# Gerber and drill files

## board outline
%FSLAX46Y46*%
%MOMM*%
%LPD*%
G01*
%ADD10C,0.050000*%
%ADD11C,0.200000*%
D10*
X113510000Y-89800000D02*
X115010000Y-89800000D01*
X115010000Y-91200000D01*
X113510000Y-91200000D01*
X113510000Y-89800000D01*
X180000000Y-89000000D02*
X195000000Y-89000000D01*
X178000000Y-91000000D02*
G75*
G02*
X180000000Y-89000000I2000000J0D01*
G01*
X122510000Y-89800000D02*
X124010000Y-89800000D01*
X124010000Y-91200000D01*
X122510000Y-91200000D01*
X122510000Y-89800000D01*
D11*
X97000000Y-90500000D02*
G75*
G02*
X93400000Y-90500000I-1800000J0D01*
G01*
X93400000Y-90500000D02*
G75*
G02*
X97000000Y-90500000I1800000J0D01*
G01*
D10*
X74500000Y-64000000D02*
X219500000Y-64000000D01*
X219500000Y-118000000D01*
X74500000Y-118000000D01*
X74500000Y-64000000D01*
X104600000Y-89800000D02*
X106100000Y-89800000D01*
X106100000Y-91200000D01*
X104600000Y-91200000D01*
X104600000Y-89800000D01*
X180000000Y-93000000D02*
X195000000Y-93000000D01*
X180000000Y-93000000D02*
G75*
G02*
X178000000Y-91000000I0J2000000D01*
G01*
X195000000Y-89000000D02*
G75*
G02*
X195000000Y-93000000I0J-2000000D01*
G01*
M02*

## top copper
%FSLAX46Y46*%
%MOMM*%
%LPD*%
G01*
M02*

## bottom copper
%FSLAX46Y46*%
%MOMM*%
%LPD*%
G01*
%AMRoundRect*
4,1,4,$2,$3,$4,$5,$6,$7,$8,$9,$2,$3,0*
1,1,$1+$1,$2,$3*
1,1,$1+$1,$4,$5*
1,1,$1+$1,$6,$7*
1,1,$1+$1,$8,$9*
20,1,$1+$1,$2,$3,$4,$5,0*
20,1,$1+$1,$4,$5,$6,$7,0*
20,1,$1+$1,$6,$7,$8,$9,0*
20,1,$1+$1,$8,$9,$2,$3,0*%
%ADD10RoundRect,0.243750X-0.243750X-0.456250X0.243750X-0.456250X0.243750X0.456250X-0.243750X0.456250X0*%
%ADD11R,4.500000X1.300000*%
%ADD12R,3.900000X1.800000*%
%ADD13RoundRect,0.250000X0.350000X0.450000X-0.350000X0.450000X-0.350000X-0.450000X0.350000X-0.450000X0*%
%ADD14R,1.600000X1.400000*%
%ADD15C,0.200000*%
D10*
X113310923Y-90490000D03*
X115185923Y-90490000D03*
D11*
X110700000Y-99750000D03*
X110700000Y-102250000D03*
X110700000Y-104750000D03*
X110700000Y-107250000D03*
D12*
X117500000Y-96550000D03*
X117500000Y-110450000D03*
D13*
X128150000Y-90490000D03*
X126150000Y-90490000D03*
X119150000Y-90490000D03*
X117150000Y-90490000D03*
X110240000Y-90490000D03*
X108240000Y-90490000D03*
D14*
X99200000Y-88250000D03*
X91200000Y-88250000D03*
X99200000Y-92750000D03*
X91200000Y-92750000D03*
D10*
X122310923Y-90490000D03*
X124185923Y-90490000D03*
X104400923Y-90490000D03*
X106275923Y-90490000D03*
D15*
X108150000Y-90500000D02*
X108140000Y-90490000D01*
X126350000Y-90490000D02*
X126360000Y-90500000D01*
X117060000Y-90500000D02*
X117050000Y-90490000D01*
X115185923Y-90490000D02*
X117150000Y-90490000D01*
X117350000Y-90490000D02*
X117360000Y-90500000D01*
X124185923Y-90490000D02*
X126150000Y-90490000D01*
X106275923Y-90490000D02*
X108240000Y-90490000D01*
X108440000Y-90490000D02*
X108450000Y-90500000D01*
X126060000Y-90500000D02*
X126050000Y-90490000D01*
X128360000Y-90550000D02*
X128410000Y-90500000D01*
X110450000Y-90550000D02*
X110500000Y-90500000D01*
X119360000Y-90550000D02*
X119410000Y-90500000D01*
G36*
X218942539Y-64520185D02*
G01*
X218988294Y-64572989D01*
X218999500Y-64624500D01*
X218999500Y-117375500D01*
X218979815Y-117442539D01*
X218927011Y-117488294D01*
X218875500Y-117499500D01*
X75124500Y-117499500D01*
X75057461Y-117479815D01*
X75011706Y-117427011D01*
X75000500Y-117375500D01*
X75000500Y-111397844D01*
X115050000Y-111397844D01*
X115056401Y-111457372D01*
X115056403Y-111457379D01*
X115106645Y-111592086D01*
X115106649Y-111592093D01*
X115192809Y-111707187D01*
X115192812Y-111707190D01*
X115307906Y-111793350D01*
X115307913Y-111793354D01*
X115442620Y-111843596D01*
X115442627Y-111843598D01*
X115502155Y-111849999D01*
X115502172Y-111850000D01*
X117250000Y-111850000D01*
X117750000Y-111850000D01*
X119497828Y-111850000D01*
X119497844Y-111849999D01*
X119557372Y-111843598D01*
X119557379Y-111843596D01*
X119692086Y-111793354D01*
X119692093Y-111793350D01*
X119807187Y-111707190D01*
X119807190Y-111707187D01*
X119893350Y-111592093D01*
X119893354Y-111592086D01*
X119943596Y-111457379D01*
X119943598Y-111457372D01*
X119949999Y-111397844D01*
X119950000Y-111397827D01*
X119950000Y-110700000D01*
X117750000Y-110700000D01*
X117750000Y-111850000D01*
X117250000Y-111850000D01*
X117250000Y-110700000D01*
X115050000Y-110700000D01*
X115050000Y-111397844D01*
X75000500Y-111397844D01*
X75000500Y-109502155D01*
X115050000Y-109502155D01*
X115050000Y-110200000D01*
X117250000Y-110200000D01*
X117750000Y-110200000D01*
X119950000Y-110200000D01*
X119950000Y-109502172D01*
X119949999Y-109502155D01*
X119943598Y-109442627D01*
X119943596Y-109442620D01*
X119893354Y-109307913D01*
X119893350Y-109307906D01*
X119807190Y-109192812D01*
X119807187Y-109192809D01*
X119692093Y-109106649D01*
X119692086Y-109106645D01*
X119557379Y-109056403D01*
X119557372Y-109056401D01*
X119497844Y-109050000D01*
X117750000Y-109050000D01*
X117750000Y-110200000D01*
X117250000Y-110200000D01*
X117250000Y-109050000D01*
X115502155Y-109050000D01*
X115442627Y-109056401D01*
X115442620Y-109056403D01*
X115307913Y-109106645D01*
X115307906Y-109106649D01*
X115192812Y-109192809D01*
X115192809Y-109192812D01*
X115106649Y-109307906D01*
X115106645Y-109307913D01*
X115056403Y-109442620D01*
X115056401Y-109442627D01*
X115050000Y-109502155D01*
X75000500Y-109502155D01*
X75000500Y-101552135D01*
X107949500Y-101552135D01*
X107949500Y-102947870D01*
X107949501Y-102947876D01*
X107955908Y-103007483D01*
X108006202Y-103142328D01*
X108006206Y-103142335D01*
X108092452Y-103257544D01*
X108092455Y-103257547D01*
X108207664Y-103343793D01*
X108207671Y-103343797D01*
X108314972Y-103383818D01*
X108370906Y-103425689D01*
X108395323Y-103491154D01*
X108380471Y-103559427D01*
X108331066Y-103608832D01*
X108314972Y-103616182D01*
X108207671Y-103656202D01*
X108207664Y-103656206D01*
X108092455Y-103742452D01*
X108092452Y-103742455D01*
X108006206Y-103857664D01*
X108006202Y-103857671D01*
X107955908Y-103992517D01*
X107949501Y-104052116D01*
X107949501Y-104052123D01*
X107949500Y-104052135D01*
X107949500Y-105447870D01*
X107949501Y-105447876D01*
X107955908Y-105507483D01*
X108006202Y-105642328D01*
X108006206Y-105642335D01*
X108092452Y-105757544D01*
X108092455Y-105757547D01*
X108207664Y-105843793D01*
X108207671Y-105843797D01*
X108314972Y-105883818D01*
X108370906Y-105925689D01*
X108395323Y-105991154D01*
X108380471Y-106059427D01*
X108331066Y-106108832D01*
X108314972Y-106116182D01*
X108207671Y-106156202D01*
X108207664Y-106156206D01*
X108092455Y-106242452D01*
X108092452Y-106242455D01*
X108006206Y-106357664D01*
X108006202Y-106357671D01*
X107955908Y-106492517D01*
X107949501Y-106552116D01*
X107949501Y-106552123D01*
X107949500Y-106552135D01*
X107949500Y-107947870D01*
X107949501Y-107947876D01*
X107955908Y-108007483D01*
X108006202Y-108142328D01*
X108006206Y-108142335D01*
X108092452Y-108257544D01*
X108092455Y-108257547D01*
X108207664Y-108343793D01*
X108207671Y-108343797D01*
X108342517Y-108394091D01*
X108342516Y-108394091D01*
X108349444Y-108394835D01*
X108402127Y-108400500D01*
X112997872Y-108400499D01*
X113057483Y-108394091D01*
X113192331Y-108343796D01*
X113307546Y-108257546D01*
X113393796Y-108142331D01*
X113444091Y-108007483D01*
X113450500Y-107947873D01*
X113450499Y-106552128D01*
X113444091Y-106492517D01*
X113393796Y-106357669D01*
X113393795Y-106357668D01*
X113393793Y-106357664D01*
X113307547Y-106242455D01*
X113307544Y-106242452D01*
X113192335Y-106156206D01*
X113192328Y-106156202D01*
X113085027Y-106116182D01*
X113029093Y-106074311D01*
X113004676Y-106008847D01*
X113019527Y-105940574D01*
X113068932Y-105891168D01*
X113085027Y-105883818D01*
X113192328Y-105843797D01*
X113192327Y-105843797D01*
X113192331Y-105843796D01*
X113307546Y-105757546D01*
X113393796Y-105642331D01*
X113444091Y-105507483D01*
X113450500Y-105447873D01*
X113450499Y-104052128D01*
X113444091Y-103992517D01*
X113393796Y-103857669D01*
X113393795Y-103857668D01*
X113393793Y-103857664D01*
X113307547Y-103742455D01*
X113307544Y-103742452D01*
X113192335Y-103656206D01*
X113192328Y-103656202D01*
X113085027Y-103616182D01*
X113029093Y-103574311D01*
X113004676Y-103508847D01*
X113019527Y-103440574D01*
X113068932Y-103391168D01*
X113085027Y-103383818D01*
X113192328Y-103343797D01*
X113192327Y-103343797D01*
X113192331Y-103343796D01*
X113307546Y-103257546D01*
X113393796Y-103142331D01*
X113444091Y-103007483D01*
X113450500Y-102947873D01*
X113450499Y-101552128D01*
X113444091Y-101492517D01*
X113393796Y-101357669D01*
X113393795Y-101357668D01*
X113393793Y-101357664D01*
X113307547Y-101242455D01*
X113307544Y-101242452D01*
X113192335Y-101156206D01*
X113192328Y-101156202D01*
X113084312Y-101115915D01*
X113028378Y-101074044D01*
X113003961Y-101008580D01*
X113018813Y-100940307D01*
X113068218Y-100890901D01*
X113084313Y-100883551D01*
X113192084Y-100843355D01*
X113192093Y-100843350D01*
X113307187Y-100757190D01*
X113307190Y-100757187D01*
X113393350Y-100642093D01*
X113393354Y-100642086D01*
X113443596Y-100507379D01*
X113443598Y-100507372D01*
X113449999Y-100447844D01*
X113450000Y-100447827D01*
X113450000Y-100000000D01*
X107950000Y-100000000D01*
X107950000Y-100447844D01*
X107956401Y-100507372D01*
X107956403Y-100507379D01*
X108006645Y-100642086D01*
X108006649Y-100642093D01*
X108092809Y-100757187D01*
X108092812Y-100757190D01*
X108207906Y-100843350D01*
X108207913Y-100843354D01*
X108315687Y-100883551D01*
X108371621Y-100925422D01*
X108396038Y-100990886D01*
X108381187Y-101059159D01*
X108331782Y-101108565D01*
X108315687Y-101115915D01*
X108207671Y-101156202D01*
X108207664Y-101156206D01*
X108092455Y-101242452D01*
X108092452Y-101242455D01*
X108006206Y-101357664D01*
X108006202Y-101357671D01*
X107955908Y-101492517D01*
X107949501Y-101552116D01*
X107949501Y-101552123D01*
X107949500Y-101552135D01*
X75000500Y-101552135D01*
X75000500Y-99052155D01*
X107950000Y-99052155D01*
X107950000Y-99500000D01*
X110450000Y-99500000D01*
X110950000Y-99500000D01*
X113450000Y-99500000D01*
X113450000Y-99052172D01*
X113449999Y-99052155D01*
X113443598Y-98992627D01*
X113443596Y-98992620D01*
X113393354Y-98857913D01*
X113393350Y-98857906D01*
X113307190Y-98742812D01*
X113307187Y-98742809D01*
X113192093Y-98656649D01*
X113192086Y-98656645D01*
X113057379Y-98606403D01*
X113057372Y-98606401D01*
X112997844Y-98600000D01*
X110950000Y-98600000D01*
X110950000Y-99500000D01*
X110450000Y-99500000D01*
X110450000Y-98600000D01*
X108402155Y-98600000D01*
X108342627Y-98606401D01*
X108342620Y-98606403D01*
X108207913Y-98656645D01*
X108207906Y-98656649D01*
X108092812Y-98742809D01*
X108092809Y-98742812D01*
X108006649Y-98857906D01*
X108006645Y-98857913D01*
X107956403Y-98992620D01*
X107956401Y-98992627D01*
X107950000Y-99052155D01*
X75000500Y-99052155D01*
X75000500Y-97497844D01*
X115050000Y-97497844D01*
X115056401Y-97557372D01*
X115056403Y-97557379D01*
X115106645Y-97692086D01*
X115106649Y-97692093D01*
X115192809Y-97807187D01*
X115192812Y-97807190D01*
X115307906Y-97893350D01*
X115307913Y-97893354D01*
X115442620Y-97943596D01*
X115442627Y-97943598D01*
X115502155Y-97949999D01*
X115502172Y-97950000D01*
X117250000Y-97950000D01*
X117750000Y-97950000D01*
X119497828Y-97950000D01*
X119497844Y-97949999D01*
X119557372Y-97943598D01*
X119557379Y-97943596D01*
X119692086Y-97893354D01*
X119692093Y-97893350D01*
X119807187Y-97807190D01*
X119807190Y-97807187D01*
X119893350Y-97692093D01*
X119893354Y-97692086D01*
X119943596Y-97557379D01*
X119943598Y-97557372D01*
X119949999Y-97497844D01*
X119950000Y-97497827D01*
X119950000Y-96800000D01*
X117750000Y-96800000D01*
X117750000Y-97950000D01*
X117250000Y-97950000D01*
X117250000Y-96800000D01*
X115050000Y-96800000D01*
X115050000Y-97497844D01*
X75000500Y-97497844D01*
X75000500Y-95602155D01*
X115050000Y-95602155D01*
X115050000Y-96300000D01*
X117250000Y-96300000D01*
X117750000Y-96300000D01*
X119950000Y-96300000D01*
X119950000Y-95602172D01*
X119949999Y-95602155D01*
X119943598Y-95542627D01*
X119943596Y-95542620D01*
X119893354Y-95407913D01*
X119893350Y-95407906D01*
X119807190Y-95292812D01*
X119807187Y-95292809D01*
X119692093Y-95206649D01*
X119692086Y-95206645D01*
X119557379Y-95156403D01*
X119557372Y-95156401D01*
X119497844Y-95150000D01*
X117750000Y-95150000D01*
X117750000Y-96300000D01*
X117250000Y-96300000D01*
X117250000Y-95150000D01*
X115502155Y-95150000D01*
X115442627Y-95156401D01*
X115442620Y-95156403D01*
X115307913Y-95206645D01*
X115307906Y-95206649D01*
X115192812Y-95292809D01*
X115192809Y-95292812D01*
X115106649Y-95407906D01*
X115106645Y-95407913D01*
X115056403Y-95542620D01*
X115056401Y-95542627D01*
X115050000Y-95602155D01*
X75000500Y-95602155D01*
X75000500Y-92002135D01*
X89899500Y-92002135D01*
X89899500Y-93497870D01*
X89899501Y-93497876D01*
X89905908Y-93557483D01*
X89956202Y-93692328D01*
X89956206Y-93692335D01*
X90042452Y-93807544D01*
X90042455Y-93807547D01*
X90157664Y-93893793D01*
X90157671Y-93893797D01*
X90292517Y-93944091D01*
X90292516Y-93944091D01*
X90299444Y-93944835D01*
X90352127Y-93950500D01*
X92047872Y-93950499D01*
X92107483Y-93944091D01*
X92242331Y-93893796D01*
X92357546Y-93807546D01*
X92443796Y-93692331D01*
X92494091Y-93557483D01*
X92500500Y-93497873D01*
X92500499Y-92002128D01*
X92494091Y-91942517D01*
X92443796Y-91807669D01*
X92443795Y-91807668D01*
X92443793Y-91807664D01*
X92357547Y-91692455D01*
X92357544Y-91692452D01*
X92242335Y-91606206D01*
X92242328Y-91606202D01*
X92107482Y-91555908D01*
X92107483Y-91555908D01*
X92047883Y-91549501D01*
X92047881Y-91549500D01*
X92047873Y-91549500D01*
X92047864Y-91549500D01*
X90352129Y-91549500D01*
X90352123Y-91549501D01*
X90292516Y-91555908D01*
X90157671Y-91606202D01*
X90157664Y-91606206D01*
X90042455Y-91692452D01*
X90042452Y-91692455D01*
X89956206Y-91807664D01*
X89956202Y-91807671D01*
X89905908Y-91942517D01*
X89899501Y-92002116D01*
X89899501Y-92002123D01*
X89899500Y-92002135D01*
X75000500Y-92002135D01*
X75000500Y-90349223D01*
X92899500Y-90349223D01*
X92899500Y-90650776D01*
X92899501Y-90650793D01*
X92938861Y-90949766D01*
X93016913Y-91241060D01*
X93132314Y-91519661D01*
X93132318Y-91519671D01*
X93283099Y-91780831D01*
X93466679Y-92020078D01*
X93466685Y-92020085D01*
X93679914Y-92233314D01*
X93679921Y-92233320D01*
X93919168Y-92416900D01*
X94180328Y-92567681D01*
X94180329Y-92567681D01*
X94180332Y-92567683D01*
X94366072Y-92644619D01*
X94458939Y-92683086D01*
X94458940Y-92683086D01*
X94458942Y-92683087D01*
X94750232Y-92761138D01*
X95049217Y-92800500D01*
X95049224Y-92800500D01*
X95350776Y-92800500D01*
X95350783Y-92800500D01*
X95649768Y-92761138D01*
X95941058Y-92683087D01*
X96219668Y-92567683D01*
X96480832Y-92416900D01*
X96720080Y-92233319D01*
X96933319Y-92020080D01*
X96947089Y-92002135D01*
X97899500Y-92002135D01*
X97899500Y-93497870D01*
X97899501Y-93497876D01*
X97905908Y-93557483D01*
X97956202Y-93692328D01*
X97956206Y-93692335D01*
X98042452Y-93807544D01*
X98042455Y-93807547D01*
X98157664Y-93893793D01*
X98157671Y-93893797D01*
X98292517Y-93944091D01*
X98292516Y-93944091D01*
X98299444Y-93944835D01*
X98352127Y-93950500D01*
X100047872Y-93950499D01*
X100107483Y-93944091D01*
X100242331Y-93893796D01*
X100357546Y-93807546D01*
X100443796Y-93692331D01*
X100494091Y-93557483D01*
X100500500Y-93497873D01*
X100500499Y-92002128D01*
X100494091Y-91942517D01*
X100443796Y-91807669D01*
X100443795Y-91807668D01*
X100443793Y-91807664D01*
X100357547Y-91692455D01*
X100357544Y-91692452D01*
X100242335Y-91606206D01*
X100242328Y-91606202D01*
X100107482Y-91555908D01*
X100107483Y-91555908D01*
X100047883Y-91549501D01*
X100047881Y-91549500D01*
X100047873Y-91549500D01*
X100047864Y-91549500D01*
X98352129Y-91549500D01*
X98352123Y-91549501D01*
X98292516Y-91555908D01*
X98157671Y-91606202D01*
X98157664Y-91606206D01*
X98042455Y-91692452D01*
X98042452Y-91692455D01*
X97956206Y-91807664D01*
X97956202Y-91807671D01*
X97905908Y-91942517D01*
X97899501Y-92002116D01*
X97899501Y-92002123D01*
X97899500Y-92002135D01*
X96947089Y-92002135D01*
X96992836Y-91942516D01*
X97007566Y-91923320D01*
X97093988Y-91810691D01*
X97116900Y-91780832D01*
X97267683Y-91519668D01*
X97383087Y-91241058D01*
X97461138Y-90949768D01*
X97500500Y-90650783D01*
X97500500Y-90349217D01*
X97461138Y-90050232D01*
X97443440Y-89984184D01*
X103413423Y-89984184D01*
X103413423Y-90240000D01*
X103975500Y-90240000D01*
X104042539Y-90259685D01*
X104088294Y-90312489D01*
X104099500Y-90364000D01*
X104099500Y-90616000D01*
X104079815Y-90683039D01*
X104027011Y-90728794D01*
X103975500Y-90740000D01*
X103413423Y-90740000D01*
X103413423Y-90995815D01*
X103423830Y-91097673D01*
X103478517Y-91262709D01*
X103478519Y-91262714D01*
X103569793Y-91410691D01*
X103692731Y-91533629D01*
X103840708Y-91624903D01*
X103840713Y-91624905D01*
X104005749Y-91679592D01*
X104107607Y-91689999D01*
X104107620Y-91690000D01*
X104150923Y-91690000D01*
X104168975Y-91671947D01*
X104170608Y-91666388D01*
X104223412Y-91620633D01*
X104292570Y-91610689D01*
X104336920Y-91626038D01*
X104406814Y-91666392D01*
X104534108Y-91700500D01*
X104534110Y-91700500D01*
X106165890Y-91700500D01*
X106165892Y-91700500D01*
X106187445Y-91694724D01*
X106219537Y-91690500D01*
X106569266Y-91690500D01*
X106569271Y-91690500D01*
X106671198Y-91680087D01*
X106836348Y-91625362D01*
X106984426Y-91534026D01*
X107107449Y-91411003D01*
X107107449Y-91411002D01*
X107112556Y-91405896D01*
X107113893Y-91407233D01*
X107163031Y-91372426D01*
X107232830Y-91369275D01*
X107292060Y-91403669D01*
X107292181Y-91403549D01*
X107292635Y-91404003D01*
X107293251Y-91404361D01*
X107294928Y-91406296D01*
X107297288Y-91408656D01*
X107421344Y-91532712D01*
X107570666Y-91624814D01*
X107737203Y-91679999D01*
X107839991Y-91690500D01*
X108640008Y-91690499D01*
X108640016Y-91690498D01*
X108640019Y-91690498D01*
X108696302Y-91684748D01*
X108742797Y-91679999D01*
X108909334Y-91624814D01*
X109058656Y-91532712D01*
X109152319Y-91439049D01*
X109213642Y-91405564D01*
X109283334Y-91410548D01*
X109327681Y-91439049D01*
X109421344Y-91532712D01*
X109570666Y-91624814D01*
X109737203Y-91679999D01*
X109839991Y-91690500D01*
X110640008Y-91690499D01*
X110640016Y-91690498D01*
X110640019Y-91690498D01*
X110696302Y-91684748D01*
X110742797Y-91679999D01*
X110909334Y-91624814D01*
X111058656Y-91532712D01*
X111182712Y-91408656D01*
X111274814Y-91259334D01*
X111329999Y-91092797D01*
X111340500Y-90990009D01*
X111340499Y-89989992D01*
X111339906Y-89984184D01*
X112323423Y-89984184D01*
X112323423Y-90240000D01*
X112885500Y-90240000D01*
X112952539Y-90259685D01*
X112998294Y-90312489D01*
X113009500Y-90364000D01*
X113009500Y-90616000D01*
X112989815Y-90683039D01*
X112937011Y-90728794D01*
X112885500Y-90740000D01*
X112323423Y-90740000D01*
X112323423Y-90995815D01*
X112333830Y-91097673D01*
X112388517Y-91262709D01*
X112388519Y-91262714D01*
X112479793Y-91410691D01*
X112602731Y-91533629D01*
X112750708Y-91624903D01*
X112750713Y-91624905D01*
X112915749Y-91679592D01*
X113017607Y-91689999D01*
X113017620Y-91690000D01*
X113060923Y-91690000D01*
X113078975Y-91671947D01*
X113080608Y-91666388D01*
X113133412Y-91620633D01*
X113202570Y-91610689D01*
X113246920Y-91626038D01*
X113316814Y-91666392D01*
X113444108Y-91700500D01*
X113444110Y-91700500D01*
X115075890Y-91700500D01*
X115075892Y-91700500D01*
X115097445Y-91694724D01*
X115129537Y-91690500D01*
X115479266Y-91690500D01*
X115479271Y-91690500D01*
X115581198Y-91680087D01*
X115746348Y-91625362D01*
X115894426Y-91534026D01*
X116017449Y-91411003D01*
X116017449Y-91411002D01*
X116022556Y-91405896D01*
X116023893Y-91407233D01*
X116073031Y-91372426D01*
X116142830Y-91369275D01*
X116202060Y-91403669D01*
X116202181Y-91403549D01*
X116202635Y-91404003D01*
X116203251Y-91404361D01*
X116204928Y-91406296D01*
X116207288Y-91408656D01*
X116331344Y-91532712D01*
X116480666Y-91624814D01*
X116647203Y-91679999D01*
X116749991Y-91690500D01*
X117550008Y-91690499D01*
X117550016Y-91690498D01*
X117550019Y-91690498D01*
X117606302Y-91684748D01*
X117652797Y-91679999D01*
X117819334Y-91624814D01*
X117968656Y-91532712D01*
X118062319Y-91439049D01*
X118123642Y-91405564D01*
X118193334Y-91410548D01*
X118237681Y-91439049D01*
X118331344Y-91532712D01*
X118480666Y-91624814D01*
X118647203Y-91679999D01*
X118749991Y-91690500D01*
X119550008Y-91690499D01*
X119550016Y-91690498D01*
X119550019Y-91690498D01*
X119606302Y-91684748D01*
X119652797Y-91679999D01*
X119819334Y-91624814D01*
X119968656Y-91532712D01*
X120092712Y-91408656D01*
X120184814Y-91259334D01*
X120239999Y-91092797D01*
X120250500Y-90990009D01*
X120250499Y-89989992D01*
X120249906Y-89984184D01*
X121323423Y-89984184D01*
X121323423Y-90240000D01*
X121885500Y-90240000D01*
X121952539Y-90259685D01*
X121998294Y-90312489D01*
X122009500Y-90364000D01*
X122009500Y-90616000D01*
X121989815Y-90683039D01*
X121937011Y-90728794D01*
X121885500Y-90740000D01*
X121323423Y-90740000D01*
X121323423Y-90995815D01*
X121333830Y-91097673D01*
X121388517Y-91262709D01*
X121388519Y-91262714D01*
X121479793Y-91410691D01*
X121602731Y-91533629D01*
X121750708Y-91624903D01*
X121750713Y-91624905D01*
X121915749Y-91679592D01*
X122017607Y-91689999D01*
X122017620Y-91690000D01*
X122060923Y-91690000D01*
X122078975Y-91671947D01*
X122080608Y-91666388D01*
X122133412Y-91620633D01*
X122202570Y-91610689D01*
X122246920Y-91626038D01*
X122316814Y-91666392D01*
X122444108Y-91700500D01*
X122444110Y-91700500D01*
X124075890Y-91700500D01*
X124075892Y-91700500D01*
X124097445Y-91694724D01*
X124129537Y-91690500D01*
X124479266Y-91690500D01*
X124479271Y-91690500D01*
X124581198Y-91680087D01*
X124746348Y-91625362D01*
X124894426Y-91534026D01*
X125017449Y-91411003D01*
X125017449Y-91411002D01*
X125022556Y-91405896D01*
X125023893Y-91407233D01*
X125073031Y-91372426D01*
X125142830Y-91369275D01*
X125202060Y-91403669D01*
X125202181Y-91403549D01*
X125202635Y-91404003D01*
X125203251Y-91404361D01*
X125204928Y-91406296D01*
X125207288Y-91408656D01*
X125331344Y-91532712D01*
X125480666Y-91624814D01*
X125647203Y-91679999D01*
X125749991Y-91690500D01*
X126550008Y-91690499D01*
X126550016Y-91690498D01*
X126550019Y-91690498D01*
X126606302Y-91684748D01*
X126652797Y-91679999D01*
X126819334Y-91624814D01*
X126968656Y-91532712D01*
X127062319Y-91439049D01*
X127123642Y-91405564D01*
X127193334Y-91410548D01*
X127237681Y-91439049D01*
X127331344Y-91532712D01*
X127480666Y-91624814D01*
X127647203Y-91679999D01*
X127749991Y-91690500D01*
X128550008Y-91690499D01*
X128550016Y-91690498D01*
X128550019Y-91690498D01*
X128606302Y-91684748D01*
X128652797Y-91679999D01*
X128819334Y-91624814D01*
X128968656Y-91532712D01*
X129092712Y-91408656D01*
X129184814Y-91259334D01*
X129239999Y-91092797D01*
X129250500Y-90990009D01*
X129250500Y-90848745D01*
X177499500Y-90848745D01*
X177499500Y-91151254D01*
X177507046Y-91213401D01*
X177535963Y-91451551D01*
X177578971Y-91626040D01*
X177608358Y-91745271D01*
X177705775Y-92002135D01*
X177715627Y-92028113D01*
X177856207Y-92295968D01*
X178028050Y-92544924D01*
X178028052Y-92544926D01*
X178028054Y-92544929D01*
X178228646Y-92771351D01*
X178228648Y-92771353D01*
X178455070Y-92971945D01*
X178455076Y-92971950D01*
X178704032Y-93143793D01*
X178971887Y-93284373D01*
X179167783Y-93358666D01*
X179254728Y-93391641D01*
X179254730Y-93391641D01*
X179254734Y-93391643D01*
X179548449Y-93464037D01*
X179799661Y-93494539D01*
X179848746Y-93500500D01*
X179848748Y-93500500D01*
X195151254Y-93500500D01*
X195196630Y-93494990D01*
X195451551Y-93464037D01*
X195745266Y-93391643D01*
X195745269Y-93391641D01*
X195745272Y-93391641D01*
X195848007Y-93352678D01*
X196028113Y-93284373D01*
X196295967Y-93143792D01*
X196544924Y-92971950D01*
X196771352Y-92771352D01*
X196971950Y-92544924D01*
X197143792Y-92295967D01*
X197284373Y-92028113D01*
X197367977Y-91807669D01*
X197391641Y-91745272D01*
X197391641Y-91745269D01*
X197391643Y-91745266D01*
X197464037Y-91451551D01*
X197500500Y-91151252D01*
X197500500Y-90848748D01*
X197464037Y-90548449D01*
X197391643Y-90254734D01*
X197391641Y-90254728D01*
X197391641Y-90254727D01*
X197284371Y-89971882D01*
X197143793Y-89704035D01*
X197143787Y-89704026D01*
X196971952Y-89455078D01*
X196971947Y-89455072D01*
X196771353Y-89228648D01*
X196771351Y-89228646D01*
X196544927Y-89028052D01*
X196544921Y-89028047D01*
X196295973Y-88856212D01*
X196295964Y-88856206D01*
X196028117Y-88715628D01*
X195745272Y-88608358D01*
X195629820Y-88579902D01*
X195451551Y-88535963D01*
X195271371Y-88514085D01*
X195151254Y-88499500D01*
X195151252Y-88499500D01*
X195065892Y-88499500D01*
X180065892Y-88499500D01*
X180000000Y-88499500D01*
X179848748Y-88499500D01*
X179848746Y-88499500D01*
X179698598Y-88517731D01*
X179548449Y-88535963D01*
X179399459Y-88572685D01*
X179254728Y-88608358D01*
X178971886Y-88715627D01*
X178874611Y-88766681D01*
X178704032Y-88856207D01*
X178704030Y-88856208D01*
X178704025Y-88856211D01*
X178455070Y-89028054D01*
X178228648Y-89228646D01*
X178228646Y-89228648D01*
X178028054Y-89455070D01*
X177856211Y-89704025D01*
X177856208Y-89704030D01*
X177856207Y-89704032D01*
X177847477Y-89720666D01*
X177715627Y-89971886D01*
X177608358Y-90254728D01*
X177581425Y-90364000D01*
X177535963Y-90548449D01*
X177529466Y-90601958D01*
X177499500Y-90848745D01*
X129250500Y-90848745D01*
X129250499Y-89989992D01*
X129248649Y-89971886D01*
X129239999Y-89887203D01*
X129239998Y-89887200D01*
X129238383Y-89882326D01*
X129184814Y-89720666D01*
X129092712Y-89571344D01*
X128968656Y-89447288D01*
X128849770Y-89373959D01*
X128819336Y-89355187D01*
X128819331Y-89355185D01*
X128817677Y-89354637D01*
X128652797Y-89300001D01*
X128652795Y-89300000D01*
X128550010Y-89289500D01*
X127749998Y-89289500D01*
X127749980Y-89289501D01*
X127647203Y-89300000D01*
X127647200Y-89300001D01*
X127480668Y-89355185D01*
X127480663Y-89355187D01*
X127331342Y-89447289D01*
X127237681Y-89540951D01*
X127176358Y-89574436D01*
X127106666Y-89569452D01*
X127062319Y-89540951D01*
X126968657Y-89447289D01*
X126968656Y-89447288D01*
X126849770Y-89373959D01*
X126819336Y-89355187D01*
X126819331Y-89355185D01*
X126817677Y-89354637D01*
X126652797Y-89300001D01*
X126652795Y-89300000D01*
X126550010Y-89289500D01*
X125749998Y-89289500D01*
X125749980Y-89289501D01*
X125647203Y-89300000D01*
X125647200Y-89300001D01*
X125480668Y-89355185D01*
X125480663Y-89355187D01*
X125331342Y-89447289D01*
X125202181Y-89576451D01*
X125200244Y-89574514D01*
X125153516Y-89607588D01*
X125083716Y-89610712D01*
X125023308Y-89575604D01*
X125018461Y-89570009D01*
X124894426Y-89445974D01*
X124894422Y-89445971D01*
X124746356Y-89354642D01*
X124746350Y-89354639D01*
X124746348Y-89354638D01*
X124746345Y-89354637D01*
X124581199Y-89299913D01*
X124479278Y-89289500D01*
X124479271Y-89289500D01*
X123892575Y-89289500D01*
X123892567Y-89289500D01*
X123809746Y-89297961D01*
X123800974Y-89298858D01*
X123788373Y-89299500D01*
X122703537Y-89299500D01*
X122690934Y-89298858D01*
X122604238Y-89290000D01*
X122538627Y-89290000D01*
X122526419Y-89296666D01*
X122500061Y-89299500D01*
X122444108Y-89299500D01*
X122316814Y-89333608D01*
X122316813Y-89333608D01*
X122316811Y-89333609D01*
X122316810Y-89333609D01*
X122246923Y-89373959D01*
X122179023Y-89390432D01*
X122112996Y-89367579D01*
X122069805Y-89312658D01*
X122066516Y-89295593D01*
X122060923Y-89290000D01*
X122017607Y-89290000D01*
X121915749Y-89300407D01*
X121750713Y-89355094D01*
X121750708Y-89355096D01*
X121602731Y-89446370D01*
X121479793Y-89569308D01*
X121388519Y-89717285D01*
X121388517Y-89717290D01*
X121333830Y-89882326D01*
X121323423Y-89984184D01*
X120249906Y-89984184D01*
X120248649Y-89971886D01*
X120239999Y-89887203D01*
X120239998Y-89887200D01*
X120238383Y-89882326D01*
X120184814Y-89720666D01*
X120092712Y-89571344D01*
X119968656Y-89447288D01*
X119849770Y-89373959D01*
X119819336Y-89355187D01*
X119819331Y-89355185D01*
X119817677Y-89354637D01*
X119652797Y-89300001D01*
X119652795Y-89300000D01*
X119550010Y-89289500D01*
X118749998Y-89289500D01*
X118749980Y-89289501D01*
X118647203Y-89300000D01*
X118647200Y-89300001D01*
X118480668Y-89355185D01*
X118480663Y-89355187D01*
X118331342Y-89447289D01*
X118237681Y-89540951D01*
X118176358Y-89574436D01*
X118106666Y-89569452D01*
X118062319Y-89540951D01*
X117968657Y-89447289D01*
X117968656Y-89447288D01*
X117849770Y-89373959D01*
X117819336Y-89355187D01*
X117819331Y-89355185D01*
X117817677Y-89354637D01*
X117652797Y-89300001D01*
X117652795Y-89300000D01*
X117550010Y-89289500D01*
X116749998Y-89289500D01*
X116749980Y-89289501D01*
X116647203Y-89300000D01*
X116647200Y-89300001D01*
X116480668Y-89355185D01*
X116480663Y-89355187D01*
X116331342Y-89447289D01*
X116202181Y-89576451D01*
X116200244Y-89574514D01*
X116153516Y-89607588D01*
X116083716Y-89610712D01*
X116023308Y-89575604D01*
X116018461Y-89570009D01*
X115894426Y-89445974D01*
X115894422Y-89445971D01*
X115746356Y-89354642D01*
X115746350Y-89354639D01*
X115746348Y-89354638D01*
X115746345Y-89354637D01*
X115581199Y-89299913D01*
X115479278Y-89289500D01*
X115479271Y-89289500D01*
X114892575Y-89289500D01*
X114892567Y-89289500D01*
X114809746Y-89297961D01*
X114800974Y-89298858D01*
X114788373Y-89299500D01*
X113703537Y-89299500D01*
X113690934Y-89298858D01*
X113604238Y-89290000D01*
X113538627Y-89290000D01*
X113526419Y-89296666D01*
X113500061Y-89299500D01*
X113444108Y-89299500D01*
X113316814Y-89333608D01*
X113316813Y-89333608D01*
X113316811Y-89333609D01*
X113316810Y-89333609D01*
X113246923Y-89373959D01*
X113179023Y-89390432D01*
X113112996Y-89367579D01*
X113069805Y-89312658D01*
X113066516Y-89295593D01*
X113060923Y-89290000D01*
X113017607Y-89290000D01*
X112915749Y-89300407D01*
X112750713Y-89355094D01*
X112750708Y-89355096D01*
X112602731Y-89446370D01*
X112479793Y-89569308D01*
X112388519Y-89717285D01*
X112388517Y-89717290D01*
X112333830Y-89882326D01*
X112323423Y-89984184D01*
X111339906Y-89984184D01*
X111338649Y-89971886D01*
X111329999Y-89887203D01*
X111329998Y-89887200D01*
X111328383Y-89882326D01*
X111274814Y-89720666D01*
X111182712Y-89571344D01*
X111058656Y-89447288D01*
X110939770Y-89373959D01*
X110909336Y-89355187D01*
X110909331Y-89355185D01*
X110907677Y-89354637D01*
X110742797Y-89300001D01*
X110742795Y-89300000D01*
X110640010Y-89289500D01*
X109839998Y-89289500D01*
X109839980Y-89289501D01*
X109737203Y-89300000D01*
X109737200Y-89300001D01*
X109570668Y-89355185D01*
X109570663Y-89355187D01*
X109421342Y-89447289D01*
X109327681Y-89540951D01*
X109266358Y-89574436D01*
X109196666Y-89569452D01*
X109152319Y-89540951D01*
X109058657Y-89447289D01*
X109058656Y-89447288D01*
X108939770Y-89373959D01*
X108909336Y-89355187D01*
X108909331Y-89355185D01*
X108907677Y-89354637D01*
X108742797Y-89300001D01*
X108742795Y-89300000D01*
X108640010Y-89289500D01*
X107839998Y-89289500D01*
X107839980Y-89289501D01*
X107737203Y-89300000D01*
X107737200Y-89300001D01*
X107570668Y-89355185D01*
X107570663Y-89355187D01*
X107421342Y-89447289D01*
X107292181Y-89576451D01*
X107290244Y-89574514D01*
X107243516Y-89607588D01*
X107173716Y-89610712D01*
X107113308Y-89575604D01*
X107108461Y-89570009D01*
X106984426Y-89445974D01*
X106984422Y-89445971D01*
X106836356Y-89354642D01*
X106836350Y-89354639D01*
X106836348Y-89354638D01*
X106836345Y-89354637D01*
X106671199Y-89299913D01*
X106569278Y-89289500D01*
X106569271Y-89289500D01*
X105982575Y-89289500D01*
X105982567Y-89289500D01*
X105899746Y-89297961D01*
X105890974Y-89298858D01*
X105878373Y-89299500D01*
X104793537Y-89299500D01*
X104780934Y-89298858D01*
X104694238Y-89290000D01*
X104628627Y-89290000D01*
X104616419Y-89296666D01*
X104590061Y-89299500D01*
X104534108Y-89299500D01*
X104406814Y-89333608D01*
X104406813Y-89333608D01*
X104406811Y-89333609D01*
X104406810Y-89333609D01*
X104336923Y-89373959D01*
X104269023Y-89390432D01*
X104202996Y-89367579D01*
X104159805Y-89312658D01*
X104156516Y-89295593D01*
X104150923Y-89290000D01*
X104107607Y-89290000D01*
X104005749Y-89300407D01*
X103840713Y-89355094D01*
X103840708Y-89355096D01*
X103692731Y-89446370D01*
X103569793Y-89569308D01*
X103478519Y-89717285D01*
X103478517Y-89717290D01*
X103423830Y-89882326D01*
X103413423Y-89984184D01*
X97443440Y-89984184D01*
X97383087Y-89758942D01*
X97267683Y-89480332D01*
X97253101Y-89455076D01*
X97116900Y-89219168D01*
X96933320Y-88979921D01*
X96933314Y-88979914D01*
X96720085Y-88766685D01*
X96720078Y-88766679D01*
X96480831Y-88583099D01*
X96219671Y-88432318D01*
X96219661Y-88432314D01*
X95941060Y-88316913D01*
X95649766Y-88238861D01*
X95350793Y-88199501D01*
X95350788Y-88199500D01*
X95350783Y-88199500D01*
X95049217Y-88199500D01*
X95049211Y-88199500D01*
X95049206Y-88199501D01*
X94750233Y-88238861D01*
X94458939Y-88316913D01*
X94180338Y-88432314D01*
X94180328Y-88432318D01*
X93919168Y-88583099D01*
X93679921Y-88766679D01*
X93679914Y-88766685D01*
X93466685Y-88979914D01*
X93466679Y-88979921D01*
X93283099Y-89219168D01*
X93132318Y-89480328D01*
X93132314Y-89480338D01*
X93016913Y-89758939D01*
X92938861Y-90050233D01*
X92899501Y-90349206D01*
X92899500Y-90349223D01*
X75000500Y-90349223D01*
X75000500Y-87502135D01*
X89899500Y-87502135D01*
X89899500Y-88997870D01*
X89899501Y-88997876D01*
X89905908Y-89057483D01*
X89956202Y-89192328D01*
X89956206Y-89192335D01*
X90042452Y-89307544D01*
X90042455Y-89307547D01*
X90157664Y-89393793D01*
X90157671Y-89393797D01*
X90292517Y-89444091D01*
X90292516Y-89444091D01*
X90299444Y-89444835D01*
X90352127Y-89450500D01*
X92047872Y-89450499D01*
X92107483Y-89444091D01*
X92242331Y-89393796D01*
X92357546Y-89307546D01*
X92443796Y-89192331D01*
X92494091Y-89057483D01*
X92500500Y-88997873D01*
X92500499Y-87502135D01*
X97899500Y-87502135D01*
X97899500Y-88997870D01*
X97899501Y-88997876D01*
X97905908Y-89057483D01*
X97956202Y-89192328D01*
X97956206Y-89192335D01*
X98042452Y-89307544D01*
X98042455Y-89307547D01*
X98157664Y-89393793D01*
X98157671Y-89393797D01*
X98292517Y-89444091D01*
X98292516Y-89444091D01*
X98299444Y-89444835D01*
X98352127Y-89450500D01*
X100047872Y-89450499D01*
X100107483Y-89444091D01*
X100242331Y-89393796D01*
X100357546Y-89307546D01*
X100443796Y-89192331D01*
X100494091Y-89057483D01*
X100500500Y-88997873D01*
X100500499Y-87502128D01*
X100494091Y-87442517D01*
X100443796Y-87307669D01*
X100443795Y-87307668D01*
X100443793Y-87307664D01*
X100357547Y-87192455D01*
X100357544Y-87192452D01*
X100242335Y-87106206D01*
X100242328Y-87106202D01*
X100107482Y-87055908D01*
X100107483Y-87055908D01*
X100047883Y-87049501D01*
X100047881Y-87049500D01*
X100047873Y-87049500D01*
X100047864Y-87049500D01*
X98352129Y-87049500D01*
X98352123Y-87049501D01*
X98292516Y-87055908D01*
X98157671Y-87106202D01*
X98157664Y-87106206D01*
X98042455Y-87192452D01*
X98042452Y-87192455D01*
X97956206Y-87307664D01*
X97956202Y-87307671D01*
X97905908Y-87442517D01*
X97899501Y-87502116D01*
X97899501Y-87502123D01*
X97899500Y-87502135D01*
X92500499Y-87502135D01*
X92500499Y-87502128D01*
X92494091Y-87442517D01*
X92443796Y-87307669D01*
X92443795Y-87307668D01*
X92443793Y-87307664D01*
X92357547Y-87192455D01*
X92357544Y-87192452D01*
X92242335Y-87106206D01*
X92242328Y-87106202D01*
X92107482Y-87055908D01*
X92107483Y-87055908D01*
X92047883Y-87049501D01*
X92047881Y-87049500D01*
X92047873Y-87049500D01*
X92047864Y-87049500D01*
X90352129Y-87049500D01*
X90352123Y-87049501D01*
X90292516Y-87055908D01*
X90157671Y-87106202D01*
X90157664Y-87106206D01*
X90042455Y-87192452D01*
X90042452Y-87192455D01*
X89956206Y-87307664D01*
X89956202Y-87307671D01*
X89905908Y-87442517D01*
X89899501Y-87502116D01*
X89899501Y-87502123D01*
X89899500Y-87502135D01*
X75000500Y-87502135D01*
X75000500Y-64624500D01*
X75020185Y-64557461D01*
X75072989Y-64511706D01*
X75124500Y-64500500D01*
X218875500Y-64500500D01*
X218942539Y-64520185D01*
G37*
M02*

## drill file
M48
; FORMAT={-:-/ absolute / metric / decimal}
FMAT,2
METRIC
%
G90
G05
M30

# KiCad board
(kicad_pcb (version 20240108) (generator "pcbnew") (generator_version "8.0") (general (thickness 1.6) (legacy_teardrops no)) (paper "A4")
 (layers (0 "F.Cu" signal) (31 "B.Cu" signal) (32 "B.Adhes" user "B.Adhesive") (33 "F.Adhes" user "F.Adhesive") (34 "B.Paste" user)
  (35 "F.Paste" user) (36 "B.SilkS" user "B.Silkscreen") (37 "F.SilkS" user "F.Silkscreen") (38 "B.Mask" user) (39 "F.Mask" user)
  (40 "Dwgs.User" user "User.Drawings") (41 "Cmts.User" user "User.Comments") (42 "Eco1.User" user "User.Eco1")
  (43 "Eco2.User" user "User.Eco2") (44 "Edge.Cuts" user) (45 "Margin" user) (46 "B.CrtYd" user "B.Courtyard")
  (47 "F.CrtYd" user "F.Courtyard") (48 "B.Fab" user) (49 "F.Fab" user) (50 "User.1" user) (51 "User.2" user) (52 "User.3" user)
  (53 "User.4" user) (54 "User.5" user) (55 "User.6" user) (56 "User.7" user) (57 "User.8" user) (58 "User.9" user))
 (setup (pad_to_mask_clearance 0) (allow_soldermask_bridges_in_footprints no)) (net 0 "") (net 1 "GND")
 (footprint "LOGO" (layer "F.Cu") (at 86 106.5)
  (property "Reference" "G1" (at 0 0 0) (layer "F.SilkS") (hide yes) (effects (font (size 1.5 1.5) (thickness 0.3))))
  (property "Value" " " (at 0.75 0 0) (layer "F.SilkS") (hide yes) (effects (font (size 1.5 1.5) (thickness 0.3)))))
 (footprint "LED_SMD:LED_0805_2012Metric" (layer "B.Cu") (at 114.248423 90.49)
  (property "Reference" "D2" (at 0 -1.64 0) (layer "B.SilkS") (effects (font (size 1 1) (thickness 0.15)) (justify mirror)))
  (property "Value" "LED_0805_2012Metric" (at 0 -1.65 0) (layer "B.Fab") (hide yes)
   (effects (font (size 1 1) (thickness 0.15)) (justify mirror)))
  (pad "1" smd roundrect (at -0.9375 0) (size 0.975 1.4) (layers "B.Cu" "B.Paste" "B.Mask") (roundrect_rratio 0.25) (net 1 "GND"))
  (pad "2" smd roundrect (at 0.9375 0) (size 0.975 1.4) (layers "B.Cu" "B.Paste" "B.Mask") (roundrect_rratio 0.25)))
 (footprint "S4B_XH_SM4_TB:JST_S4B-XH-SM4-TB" (layer "B.Cu") (at 117.5 103.5 -90)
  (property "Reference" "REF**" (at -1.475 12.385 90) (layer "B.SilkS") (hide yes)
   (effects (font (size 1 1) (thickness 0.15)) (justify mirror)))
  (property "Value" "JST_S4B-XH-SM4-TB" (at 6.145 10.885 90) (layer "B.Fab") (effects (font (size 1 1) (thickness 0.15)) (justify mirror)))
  (pad "1" smd rect (at -3.75 6.8 270) (size 1.3 4.5) (layers "B.Cu" "B.Paste" "B.Mask") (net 1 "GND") (solder_mask_margin 0.102))
  (pad "2" smd rect (at -1.25 6.8 270) (size 1.3 4.5) (layers "B.Cu" "B.Paste" "B.Mask") (solder_mask_margin 0.102))
  (pad "3" smd rect (at 1.25 6.8 270) (size 1.3 4.5) (layers "B.Cu" "B.Paste" "B.Mask") (solder_mask_margin 0.102))
  (pad "4" smd rect (at 3.75 6.8 270) (size 1.3 4.5) (layers "B.Cu" "B.Paste" "B.Mask") (solder_mask_margin 0.102))
  (pad "SH1" smd rect (at -6.95 0 270) (size 1.8 3.9) (layers "B.Cu" "B.Paste" "B.Mask") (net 1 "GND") (solder_mask_margin 0.102))
  (pad "SH2" smd rect (at 6.95 0 270) (size 1.8 3.9) (layers "B.Cu" "B.Paste" "B.Mask") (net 1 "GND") (solder_mask_margin 0.102)))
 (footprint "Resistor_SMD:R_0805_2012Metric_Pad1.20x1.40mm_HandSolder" (layer "B.Cu") (at 127.15 90.49 180)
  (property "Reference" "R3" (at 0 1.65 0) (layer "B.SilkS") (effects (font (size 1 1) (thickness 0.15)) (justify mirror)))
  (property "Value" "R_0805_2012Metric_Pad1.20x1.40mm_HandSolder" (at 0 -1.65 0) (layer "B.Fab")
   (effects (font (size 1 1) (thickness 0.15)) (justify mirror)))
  (pad "1" smd roundrect (at -1 0 180) (size 1.2 1.4) (layers "B.Cu" "B.Paste" "B.Mask") (roundrect_rratio 0.208333))
  (pad "2" smd roundrect (at 1 0 180) (size 1.2 1.4) (layers "B.Cu" "B.Paste" "B.Mask") (roundrect_rratio 0.208333)))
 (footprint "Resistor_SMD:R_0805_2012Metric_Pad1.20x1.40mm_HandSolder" (layer "B.Cu") (at 118.15 90.49 180)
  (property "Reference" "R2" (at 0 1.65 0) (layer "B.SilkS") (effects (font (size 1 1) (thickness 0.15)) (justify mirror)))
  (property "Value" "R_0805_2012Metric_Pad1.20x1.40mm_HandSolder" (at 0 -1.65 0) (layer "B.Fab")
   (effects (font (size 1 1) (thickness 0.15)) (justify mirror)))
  (pad "1" smd roundrect (at -1 0 180) (size 1.2 1.4) (layers "B.Cu" "B.Paste" "B.Mask") (roundrect_rratio 0.208333))
  (pad "2" smd roundrect (at 1 0 180) (size 1.2 1.4) (layers "B.Cu" "B.Paste" "B.Mask") (roundrect_rratio 0.208333)))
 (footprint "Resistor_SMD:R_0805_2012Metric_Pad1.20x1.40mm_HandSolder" (layer "B.Cu") (at 109.24 90.49 180)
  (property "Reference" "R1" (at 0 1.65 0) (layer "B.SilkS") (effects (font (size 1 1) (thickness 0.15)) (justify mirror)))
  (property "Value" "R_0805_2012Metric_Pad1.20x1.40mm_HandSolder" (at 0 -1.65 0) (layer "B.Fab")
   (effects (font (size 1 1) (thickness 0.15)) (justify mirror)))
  (pad "1" smd roundrect (at -1 0 180) (size 1.2 1.4) (layers "B.Cu" "B.Paste" "B.Mask") (roundrect_rratio 0.208333))
  (pad "2" smd roundrect (at 1 0 180) (size 1.2 1.4) (layers "B.Cu" "B.Paste" "B.Mask") (roundrect_rratio 0.208333)))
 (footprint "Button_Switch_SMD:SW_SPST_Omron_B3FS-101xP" (layer "B.Cu") (at 95.2 90.5 180)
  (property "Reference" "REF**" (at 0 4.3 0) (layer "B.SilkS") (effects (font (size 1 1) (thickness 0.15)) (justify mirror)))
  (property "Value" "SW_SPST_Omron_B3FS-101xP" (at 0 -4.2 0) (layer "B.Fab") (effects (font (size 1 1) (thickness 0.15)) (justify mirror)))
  (pad "1" smd rect (at -4 2.25) (size 1.6 1.4) (layers "B.Cu" "B.Paste" "B.Mask"))
  (pad "1" smd rect (at 4 2.25) (size 1.6 1.4) (layers "B.Cu" "B.Paste" "B.Mask"))
  (pad "2" smd rect (at -4 -2.25) (size 1.6 1.4) (layers "B.Cu" "B.Paste" "B.Mask"))
  (pad "2" smd rect (at 4 -2.25) (size 1.6 1.4) (layers "B.Cu" "B.Paste" "B.Mask")))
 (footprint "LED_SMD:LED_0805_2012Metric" (layer "B.Cu") (at 123.248423 90.49)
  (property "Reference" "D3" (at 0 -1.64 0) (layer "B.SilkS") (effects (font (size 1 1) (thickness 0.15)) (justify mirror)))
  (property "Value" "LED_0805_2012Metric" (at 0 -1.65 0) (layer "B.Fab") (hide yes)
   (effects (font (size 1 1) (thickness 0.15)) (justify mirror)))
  (pad "1" smd roundrect (at -0.9375 0) (size 0.975 1.4) (layers "B.Cu" "B.Paste" "B.Mask") (roundrect_rratio 0.25) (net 1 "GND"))
  (pad "2" smd roundrect (at 0.9375 0) (size 0.975 1.4) (layers "B.Cu" "B.Paste" "B.Mask") (roundrect_rratio 0.25)))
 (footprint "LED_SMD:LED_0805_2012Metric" (layer "B.Cu") (at 105.338423 90.49)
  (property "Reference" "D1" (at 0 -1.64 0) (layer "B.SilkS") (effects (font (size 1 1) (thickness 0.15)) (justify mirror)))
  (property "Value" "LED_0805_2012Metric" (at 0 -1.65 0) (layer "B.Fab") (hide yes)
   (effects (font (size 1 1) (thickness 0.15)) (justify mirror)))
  (pad "1" smd roundrect (at -0.9375 0) (size 0.975 1.4) (layers "B.Cu" "B.Paste" "B.Mask") (roundrect_rratio 0.25) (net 1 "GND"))
  (pad "2" smd roundrect (at 0.9375 0) (size 0.975 1.4) (layers "B.Cu" "B.Paste" "B.Mask") (roundrect_rratio 0.25)))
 (gr_rect (start 113.51 89.8) (end 115.01 91.2) (stroke (width 0.05) (type default)) (fill none) (layer "Edge.Cuts"))
 (gr_line (start 180 89) (end 195 89) (stroke (width 0.05) (type default)) (layer "Edge.Cuts"))
 (gr_arc (start 178 91) (mid 178.585786 89.585786) (end 180 89) (stroke (width 0.05) (type default)) (layer "Edge.Cuts"))
 (gr_rect (start 122.51 89.8) (end 124.01 91.2) (stroke (width 0.05) (type default)) (fill none) (layer "Edge.Cuts"))
 (gr_circle (center 95.2 90.5) (end 97 90.5) (stroke (width 0.2) (type default)) (fill none) (layer "Edge.Cuts"))
 (gr_rect (start 74.5 64) (end 219.5 118) (stroke (width 0.05) (type default)) (fill none) (layer "Edge.Cuts"))
 (gr_rect (start 104.6 89.8) (end 106.1 91.2) (stroke (width 0.05) (type default)) (fill none) (layer "Edge.Cuts"))
 (gr_line (start 180 93) (end 195 93) (stroke (width 0.05) (type default)) (layer "Edge.Cuts"))
 (gr_arc (start 180 93) (mid 178.585786 92.414214) (end 178 91) (stroke (width 0.05) (type default)) (layer "Edge.Cuts"))
 (gr_arc (start 195 89) (mid 197 91) (end 195 93) (stroke (width 0.05) (type default)) (layer "Edge.Cuts"))
 (segment (start 108.15 90.5) (end 108.14 90.49) (width 0.2) (layer "B.Cu") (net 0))
 (segment (start 126.35 90.49) (end 126.36 90.5) (width 0.2) (layer "B.Cu") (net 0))
 (segment (start 117.06 90.5) (end 117.05 90.49) (width 0.2) (layer "B.Cu") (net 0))
 (segment (start 115.185923 90.49) (end 117.15 90.49) (width 0.2) (layer "B.Cu") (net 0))
 (segment (start 117.35 90.49) (end 117.36 90.5) (width 0.2) (layer "B.Cu") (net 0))
 (segment (start 124.185923 90.49) (end 126.15 90.49) (width 0.2) (layer "B.Cu") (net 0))
 (segment (start 106.275923 90.49) (end 108.24 90.49) (width 0.2) (layer "B.Cu") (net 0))
 (segment (start 108.44 90.49) (end 108.45 90.5) (width 0.2) (layer "B.Cu") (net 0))
 (segment (start 126.06 90.5) (end 126.05 90.49) (width 0.2) (layer "B.Cu") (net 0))
 (segment (start 128.36 90.55) (end 128.41 90.5) (width 0.2) (layer "B.Cu") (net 1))
 (segment (start 110.45 90.55) (end 110.5 90.5) (width 0.2) (layer "B.Cu") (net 1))
 (segment (start 119.36 90.55) (end 119.41 90.5) (width 0.2) (layer "B.Cu") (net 1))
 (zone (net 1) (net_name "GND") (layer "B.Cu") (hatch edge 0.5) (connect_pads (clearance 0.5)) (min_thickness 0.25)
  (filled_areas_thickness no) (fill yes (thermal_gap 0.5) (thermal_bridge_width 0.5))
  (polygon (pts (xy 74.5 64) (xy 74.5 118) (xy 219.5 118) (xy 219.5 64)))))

